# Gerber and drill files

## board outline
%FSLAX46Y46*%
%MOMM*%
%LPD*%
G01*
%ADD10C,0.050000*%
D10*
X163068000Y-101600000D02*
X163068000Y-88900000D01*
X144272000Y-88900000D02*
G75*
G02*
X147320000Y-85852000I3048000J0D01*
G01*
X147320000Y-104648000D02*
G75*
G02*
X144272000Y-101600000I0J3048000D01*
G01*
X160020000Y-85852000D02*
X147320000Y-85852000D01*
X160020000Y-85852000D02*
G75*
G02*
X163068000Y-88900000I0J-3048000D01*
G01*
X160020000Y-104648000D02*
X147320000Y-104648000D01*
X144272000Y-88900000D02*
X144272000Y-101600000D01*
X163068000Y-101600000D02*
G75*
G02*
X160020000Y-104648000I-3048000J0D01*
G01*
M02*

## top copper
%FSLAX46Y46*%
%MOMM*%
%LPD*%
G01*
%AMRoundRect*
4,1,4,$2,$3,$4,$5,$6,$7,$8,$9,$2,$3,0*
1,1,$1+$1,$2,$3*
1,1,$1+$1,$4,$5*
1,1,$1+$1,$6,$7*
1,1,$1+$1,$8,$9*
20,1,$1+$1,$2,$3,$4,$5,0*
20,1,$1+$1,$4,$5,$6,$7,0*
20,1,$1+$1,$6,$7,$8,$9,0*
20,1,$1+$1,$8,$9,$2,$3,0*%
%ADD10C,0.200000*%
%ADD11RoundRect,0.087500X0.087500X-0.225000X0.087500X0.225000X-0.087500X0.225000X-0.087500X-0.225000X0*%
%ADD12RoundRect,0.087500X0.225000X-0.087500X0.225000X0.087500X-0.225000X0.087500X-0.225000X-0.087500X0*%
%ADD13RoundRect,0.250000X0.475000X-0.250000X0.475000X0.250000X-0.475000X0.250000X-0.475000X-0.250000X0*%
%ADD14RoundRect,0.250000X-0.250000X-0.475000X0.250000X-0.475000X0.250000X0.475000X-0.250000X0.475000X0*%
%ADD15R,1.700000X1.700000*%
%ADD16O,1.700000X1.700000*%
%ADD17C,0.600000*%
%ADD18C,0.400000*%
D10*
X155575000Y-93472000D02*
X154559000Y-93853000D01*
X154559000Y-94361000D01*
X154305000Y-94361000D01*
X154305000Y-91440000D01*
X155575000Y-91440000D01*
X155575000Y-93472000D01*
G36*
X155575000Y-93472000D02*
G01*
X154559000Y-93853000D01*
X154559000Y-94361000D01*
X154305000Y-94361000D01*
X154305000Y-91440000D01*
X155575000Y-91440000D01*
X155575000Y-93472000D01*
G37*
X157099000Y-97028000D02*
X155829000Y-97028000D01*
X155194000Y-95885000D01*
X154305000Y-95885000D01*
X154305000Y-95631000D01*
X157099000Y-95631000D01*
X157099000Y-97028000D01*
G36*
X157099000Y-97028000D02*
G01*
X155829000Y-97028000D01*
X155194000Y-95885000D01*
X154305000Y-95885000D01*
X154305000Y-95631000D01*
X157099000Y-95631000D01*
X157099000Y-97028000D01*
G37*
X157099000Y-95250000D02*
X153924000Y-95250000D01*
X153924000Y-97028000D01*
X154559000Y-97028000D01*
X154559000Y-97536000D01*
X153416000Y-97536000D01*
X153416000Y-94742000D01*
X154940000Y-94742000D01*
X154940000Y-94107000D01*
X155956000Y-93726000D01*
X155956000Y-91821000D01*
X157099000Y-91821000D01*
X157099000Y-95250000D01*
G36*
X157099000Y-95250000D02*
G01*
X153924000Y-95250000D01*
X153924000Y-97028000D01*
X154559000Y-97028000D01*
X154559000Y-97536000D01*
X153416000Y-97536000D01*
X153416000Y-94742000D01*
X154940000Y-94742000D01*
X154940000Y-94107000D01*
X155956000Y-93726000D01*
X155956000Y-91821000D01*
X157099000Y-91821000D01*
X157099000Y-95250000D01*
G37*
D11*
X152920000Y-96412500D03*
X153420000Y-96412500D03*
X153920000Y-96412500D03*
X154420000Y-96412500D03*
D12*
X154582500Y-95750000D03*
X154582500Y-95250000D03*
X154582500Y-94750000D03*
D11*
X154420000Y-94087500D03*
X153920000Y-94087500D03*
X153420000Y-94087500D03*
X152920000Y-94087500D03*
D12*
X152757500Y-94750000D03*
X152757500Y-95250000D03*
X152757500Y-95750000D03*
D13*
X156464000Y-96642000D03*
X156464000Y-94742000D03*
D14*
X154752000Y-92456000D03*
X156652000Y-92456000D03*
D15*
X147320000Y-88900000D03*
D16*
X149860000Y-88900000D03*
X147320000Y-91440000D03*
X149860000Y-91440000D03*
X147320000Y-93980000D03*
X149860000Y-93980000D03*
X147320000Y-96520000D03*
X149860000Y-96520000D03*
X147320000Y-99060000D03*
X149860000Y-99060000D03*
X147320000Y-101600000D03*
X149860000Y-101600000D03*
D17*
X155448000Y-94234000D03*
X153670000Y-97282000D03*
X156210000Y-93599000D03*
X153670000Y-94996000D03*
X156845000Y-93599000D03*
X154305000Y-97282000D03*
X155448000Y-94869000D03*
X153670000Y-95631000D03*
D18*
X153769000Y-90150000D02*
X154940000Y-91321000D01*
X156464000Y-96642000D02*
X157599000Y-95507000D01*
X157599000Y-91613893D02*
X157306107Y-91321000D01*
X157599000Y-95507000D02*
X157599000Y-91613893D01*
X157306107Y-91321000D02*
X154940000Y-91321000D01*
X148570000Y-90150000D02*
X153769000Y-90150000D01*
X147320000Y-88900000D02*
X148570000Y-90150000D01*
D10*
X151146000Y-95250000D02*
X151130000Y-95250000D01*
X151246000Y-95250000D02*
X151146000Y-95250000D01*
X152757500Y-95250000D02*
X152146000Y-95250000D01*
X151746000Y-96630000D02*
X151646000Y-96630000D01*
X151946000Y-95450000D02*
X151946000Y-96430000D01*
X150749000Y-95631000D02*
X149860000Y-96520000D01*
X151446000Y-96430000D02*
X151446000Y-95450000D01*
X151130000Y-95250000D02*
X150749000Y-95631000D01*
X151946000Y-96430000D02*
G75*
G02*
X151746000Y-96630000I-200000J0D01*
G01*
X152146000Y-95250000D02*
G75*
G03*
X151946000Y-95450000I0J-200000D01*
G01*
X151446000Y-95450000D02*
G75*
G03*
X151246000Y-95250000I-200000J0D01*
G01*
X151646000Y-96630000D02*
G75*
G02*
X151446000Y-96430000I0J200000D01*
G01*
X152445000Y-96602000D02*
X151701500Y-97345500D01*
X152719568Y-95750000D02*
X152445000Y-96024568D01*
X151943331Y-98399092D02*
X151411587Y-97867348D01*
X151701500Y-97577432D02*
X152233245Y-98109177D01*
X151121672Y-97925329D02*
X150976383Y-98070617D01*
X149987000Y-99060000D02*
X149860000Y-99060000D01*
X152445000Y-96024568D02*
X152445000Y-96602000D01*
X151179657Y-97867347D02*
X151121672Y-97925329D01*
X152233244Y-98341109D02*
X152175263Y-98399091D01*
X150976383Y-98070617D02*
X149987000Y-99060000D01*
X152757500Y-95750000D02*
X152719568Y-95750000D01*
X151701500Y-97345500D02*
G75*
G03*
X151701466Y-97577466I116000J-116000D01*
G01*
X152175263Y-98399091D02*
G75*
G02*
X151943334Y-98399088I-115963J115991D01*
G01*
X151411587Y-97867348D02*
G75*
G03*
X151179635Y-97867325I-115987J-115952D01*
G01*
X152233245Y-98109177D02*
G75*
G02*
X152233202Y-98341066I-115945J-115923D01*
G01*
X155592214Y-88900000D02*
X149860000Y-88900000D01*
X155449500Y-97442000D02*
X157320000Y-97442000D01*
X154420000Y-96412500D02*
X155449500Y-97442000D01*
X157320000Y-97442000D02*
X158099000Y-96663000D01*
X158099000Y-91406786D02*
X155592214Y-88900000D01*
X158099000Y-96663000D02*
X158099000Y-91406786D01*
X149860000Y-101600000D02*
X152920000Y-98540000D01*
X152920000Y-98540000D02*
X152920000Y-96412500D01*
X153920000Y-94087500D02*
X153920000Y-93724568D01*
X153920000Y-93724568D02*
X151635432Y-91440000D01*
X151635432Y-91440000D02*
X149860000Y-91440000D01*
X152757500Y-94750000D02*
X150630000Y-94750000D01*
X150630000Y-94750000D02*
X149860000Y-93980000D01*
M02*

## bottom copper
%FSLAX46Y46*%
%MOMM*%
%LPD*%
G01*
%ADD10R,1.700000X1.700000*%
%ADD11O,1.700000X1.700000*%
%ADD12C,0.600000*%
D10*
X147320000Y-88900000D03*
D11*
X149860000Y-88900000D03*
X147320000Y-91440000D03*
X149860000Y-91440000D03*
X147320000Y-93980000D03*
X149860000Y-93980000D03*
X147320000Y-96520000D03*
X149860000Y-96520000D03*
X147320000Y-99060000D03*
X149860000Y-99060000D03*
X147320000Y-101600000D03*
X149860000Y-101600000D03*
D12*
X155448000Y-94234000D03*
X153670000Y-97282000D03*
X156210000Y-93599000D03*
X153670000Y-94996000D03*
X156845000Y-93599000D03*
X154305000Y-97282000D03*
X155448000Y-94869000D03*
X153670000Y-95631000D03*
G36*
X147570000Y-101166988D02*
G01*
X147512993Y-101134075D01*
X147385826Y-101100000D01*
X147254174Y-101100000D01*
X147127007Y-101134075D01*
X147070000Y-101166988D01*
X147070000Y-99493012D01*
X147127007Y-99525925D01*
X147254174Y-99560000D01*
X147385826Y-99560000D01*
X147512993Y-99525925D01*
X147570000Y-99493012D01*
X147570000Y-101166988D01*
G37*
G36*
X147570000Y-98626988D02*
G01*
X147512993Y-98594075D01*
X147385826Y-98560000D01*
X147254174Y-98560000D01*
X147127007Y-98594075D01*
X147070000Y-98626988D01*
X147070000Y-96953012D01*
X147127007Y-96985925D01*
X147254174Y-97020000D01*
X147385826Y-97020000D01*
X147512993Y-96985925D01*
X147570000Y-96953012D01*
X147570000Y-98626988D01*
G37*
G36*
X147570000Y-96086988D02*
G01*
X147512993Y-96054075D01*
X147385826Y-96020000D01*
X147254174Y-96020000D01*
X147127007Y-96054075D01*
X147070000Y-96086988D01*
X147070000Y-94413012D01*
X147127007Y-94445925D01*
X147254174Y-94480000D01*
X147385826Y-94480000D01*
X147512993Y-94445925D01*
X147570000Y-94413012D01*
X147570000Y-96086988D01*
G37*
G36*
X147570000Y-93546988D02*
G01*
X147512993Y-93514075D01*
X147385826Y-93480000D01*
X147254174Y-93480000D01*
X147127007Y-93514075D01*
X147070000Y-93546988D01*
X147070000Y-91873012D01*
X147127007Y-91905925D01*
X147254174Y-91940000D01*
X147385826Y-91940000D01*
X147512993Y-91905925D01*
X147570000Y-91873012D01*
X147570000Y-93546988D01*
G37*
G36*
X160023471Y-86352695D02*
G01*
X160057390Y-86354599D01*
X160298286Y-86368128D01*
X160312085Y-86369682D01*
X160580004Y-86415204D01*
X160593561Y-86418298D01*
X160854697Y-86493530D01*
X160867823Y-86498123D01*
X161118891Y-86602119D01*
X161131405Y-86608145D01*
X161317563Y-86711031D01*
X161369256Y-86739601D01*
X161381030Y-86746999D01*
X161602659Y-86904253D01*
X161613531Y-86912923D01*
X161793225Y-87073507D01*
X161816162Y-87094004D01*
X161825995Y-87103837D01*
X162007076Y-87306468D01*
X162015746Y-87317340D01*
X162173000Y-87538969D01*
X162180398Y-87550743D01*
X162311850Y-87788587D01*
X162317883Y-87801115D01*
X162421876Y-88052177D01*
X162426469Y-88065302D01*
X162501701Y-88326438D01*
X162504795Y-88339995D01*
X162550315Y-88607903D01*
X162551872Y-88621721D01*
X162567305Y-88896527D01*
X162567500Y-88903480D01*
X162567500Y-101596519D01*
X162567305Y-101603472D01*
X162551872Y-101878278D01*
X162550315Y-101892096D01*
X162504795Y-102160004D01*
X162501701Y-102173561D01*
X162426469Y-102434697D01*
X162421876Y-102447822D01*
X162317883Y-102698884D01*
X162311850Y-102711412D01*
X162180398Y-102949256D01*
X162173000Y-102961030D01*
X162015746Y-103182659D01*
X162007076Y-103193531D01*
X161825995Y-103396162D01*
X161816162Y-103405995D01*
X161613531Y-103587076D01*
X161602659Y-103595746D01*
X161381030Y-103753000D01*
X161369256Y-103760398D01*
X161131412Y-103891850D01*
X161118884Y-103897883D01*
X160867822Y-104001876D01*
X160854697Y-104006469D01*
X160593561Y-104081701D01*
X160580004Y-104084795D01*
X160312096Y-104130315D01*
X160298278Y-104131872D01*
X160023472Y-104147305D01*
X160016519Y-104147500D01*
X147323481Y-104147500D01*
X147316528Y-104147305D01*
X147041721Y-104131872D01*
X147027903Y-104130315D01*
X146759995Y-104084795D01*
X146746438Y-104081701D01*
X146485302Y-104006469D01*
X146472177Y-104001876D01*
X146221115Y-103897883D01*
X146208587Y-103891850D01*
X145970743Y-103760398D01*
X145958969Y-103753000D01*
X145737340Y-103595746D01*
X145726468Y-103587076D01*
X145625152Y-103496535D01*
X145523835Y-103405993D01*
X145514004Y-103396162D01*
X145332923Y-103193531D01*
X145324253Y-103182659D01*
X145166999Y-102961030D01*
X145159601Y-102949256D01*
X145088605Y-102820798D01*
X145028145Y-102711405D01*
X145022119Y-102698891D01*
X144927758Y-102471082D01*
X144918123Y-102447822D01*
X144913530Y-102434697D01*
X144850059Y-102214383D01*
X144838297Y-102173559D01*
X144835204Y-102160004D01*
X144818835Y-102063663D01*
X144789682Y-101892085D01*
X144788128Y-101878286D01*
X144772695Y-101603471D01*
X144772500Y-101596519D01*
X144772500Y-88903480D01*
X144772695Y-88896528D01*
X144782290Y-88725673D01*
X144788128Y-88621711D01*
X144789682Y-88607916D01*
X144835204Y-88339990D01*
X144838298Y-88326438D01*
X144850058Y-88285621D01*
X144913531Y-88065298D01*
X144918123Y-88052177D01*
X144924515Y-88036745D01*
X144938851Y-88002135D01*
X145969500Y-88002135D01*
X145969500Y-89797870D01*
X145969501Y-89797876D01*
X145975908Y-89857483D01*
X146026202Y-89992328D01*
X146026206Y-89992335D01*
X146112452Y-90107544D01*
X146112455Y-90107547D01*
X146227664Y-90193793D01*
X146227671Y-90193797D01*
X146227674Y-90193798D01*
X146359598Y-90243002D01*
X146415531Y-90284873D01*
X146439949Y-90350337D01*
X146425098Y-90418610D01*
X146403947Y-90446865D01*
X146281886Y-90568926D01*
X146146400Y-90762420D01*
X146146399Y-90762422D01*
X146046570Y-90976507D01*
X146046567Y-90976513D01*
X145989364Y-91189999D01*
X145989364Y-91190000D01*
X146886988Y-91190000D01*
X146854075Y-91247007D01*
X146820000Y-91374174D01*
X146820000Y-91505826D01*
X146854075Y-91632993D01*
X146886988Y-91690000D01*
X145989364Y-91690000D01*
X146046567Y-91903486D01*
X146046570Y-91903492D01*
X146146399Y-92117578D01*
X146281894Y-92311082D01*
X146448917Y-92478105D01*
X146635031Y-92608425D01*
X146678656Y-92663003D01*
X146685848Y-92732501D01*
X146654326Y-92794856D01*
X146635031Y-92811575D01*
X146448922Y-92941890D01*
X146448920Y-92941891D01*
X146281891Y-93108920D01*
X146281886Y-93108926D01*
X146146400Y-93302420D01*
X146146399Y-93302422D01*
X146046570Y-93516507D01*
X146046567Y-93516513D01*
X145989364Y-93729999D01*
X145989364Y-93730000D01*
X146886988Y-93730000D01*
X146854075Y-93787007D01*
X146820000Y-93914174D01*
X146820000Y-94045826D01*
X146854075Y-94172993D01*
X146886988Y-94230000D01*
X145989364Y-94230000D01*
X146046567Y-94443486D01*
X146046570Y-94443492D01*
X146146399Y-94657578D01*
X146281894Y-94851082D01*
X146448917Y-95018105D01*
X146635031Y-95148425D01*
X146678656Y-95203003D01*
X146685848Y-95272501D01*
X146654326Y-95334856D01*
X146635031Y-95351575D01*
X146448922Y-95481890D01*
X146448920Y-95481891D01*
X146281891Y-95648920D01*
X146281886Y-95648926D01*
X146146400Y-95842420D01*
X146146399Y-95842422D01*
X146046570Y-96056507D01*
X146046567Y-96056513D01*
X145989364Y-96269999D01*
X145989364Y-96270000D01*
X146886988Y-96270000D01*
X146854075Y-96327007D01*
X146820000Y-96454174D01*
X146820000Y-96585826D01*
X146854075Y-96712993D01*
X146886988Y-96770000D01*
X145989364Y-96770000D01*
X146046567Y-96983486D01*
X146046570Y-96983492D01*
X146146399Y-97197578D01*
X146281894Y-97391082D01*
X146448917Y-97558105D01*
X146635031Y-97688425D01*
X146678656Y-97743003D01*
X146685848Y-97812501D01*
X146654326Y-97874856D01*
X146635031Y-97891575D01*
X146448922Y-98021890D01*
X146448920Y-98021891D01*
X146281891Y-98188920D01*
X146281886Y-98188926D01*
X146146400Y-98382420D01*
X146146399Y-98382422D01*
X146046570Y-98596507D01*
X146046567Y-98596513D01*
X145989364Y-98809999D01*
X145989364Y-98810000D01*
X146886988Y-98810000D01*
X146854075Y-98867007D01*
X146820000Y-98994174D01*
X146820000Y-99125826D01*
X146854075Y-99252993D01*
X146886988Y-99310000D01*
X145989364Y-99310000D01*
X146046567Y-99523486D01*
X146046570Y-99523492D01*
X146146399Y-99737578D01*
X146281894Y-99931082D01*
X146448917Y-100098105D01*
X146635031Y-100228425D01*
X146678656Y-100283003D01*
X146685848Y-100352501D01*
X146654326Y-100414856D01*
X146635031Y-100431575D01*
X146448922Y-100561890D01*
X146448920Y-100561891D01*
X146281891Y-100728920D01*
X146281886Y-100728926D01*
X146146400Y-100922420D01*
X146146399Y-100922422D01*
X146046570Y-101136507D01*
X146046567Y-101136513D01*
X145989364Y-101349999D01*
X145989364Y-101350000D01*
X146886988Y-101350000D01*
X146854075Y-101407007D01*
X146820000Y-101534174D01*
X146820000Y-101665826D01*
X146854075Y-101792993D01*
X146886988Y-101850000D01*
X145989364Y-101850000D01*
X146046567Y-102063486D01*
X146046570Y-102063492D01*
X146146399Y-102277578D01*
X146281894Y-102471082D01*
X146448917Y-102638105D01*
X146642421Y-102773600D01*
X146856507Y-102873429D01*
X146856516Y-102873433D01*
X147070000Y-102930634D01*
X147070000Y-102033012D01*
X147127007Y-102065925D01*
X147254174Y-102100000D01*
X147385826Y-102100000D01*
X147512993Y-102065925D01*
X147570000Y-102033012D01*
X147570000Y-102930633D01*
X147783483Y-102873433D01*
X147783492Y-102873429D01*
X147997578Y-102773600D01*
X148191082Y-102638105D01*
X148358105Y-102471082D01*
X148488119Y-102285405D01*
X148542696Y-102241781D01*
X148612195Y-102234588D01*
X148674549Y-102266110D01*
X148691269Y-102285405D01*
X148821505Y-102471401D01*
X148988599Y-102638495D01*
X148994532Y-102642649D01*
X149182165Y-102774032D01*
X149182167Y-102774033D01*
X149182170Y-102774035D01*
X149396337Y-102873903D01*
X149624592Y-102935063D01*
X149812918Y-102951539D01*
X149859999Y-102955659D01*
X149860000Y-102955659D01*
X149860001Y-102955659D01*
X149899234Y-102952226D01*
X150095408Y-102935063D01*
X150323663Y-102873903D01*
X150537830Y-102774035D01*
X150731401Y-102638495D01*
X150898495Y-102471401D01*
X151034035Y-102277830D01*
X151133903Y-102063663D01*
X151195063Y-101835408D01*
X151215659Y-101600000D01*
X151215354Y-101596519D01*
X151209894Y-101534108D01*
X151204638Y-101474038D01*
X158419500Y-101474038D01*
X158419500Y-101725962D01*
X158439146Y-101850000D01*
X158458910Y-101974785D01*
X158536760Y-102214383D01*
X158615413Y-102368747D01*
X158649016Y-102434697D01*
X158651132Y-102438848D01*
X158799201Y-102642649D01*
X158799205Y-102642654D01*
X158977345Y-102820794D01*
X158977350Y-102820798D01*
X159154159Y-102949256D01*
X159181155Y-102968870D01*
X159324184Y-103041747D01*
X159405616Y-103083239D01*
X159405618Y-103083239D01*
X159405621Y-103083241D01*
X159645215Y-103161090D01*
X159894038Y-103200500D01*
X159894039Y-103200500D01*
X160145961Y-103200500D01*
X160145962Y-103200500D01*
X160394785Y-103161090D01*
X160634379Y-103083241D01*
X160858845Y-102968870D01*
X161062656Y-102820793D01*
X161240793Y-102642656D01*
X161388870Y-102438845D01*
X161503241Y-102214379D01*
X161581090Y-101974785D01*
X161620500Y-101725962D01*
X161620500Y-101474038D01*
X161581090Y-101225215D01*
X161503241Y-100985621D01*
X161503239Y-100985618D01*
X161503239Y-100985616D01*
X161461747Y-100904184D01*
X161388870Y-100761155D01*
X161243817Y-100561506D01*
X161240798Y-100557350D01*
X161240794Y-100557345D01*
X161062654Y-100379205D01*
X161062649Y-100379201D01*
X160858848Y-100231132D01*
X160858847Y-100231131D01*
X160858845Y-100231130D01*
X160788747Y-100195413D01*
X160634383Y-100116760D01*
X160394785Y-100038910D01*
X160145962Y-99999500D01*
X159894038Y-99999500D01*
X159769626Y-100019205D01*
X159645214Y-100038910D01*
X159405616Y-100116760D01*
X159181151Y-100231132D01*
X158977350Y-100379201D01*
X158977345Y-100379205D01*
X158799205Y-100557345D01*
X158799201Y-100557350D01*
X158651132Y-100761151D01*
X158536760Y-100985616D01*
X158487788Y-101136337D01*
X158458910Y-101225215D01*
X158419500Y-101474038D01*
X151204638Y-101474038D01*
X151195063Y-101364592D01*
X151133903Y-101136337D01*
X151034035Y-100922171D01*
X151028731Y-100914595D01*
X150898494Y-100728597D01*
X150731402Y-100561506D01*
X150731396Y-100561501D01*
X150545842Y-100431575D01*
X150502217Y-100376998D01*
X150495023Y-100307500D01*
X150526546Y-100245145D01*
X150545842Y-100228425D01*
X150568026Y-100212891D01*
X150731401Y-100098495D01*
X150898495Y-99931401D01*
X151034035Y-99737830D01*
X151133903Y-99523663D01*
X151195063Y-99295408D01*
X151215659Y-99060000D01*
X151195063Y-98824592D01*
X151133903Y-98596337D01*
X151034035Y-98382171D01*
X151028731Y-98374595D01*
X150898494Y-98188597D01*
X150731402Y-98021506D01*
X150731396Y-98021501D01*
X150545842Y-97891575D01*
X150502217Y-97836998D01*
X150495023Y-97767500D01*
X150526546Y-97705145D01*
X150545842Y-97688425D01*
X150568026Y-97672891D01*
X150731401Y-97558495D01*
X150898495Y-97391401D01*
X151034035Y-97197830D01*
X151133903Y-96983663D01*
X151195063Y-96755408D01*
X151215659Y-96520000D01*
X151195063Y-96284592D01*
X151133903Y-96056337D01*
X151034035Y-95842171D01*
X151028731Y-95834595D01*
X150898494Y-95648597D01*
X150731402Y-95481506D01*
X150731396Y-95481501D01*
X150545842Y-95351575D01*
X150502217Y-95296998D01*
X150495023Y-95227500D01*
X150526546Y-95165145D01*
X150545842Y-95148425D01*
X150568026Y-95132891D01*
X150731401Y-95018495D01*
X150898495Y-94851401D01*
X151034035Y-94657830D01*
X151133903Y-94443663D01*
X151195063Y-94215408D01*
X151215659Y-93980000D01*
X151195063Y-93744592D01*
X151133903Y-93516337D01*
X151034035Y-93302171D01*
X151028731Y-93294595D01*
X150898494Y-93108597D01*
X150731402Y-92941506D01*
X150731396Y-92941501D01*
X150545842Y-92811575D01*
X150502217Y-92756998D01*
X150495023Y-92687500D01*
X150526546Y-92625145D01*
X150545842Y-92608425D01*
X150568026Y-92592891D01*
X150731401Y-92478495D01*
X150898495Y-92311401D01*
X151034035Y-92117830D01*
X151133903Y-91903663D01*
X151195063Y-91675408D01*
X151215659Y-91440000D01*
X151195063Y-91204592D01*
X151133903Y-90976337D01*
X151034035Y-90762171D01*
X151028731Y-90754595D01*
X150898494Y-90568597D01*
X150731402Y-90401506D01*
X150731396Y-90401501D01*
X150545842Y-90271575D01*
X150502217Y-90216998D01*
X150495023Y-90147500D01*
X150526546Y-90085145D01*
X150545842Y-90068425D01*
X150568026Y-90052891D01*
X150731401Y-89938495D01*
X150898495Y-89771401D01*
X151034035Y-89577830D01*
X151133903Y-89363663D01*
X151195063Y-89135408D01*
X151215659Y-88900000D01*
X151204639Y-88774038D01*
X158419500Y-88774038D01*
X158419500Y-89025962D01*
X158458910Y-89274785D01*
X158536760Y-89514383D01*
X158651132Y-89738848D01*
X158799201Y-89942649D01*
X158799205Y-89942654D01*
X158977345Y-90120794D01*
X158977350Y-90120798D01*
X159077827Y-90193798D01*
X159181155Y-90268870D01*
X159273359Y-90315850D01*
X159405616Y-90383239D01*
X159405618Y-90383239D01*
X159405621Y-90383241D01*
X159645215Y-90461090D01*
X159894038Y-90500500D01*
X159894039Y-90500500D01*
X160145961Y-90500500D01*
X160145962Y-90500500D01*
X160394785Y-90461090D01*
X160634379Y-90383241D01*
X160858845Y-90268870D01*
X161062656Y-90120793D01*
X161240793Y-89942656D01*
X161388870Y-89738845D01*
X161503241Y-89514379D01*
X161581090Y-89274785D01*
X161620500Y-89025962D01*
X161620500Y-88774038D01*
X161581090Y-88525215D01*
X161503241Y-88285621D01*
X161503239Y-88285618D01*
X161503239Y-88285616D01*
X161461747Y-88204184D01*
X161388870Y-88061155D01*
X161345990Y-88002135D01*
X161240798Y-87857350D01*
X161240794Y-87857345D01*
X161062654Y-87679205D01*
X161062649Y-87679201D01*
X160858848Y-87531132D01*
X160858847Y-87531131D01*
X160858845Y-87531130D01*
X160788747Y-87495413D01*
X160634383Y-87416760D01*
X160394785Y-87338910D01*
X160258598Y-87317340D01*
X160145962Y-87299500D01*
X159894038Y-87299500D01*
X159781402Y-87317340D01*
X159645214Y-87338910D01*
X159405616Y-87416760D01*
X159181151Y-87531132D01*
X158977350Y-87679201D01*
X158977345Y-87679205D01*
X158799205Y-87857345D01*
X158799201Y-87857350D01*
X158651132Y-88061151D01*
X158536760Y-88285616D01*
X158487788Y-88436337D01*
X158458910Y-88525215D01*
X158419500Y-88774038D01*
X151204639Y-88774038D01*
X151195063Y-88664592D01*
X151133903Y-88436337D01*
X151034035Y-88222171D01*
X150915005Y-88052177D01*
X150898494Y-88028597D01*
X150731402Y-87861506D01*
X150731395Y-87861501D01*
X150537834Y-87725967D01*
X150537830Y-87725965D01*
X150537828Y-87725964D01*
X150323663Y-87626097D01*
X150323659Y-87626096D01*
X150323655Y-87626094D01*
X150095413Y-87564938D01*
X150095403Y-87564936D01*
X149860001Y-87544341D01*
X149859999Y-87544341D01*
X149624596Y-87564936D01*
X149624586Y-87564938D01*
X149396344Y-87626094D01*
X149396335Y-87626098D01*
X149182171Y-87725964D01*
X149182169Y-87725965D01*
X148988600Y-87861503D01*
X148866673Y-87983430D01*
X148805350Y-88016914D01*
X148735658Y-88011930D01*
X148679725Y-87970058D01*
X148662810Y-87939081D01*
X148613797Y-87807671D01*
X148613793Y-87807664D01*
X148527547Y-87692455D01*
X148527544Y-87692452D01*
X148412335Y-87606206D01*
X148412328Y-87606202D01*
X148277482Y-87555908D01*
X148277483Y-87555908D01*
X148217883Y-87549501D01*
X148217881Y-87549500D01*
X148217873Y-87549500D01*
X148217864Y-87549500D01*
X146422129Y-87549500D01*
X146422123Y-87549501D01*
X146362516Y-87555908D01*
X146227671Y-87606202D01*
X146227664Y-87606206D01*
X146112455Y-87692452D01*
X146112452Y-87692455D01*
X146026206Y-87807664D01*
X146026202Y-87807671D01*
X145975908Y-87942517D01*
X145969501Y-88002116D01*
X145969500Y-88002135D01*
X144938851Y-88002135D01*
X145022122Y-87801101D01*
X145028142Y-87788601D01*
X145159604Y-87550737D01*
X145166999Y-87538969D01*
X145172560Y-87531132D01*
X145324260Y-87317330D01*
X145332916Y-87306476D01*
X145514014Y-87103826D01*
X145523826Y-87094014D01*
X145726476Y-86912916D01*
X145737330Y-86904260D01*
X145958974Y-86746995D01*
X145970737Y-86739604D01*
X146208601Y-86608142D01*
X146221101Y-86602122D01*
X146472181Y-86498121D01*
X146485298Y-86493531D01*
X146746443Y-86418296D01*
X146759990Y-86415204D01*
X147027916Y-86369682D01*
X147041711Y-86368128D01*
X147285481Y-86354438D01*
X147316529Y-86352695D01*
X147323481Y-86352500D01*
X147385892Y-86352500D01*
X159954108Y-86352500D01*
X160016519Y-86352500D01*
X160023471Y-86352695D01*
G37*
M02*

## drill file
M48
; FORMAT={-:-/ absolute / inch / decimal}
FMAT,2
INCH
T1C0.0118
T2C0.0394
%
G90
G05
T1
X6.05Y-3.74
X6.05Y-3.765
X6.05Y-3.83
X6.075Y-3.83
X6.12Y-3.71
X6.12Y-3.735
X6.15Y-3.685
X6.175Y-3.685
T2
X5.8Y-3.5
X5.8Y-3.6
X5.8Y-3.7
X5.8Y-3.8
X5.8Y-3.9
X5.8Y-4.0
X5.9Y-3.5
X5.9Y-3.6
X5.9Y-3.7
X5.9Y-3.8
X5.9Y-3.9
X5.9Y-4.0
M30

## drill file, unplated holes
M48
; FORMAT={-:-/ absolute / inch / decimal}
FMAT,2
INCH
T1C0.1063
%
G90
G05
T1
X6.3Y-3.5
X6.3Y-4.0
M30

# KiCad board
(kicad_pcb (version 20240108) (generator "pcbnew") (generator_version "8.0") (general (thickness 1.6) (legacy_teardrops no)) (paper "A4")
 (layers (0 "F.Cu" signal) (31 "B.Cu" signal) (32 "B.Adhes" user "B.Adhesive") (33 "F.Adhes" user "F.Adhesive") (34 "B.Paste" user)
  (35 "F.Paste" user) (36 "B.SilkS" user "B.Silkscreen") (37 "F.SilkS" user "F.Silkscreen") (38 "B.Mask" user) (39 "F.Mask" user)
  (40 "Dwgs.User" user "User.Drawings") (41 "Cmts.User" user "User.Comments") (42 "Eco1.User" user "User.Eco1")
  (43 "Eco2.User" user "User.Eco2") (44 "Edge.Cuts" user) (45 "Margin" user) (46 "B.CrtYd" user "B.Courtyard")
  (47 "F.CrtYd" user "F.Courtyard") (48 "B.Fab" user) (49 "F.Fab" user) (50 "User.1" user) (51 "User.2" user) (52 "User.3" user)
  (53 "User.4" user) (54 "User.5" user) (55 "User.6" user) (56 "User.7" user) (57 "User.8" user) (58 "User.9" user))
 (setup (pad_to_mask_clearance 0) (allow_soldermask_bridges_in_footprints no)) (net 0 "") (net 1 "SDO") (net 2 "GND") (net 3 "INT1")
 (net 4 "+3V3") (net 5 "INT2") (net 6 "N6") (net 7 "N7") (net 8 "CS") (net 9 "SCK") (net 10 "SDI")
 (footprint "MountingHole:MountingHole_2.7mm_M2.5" (layer "F.Cu") (at 160.02 101.6)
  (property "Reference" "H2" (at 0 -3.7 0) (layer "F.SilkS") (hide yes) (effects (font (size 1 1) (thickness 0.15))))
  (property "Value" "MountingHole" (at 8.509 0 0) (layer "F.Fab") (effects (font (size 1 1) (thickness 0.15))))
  (pad "" np_thru_hole circle (at 0 0) (size 2.7 2.7) (drill 2.7) (layers "*.Cu" "*.Mask")))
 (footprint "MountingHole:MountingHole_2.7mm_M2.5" (layer "F.Cu") (at 160.02 88.9)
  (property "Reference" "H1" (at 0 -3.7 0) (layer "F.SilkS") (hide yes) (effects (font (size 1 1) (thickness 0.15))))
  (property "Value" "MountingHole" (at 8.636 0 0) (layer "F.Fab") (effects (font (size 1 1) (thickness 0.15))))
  (pad "" np_thru_hole circle (at 0 0) (size 2.7 2.7) (drill 2.7) (layers "*.Cu" "*.Mask")))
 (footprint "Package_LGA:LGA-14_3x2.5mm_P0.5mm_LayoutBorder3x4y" (layer "F.Cu") (at 153.67 95.25 90)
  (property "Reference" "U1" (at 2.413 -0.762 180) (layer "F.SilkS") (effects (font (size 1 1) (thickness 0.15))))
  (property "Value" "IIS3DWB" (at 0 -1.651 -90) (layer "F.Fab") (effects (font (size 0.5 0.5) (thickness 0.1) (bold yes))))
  (pad "1" smd roundrect (at -1.1625 -0.75 90) (size 0.625 0.35) (layers "F.Cu" "F.Paste" "F.Mask") (roundrect_rratio 0.25) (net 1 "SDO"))
  (pad "2" smd roundrect (at -1.1625 -0.25 90) (size 0.625 0.35) (layers "F.Cu" "F.Paste" "F.Mask") (roundrect_rratio 0.25) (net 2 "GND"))
  (pad "3" smd roundrect (at -1.1625 0.25 90) (size 0.625 0.35) (layers "F.Cu" "F.Paste" "F.Mask") (roundrect_rratio 0.25) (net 2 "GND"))
  (pad "4" smd roundrect (at -1.1625 0.75 90) (size 0.625 0.35) (layers "F.Cu" "F.Paste" "F.Mask") (roundrect_rratio 0.25) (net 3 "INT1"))
  (pad "5" smd roundrect (at -0.5 0.9125 90) (size 0.35 0.625) (layers "F.Cu" "F.Paste" "F.Mask") (roundrect_rratio 0.25) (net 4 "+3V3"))
  (pad "6" smd roundrect (at 0 0.9125 90) (size 0.35 0.625) (layers "F.Cu" "F.Paste" "F.Mask") (roundrect_rratio 0.25) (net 2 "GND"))
  (pad "7" smd roundrect (at 0.5 0.9125 90) (size 0.35 0.625) (layers "F.Cu" "F.Paste" "F.Mask") (roundrect_rratio 0.25) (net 2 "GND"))
  (pad "8" smd roundrect (at 1.1625 0.75 90) (size 0.625 0.35) (layers "F.Cu" "F.Paste" "F.Mask") (roundrect_rratio 0.25) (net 4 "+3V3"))
  (pad "9" smd roundrect (at 1.1625 0.25 90) (size 0.625 0.35) (layers "F.Cu" "F.Paste" "F.Mask") (roundrect_rratio 0.25) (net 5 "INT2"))
  (pad "10" smd roundrect (at 1.1625 -0.25 90) (size 0.625 0.35) (layers "F.Cu" "F.Paste" "F.Mask") (roundrect_rratio 0.25) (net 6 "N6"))
  (pad "11" smd roundrect (at 1.1625 -0.75 90) (size 0.625 0.35) (layers "F.Cu" "F.Paste" "F.Mask") (roundrect_rratio 0.25) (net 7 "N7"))
  (pad "12" smd roundrect (at 0.5 -0.9125 90) (size 0.35 0.625) (layers "F.Cu" "F.Paste" "F.Mask") (roundrect_rratio 0.25) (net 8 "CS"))
  (pad "13" smd roundrect (at 0 -0.9125 90) (size 0.35 0.625) (layers "F.Cu" "F.Paste" "F.Mask") (roundrect_rratio 0.25) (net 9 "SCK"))
  (pad "14" smd roundrect (at -0.5 -0.9125 90) (size 0.35 0.625) (layers "F.Cu" "F.Paste" "F.Mask") (roundrect_rratio 0.25) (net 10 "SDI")))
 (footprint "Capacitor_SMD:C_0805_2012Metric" (layer "F.Cu") (at 156.464 95.692 90)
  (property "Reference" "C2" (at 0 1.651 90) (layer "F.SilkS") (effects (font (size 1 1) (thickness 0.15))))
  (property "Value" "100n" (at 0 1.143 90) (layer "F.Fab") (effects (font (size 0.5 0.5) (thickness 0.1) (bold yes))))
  (pad "1" smd roundrect (at -0.95 0 90) (size 1 1.45) (layers "F.Cu" "F.Paste" "F.Mask") (roundrect_rratio 0.25) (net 4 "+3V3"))
  (pad "2" smd roundrect (at 0.95 0 90) (size 1 1.45) (layers "F.Cu" "F.Paste" "F.Mask") (roundrect_rratio 0.25) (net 2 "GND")))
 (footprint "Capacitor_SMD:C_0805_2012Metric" (layer "F.Cu") (at 155.702 92.456)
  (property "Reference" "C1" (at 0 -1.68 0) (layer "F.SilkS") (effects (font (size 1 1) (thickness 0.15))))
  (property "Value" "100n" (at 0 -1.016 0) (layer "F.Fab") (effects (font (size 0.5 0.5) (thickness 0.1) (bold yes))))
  (pad "1" smd roundrect (at -0.95 0) (size 1 1.45) (layers "F.Cu" "F.Paste" "F.Mask") (roundrect_rratio 0.25) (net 4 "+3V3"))
  (pad "2" smd roundrect (at 0.95 0) (size 1 1.45) (layers "F.Cu" "F.Paste" "F.Mask") (roundrect_rratio 0.25) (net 2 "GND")))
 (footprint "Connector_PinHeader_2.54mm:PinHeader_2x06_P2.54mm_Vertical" (layer "F.Cu") (at 147.32 88.9)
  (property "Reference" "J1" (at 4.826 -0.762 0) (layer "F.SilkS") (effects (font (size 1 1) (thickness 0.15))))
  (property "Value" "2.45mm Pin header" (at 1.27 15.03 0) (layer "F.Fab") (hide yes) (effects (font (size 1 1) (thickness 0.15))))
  (pad "1" thru_hole rect (at 0 0) (size 1.7 1.7) (drill 1) (layers "*.Cu" "*.Mask") (remove_unused_layers no) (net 4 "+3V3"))
  (pad "2" thru_hole oval (at 2.54 0) (size 1.7 1.7) (drill 1) (layers "*.Cu" "*.Mask") (remove_unused_layers no) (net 3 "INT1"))
  (pad "3" thru_hole oval (at 0 2.54) (size 1.7 1.7) (drill 1) (layers "*.Cu" "*.Mask") (remove_unused_layers no) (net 2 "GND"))
  (pad "4" thru_hole oval (at 2.54 2.54) (size 1.7 1.7) (drill 1) (layers "*.Cu" "*.Mask") (remove_unused_layers no) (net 5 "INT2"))
  (pad "5" thru_hole oval (at 0 5.08) (size 1.7 1.7) (drill 1) (layers "*.Cu" "*.Mask") (remove_unused_layers no) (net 2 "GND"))
  (pad "6" thru_hole oval (at 2.54 5.08) (size 1.7 1.7) (drill 1) (layers "*.Cu" "*.Mask") (remove_unused_layers no) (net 8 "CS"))
  (pad "7" thru_hole oval (at 0 7.62) (size 1.7 1.7) (drill 1) (layers "*.Cu" "*.Mask") (remove_unused_layers no) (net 2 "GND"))
  (pad "8" thru_hole oval (at 2.54 7.62) (size 1.7 1.7) (drill 1) (layers "*.Cu" "*.Mask") (remove_unused_layers no) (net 9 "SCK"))
  (pad "9" thru_hole oval (at 0 10.16) (size 1.7 1.7) (drill 1) (layers "*.Cu" "*.Mask") (remove_unused_layers no) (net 2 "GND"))
  (pad "10" thru_hole oval (at 2.54 10.16) (size 1.7 1.7) (drill 1) (layers "*.Cu" "*.Mask") (remove_unused_layers no) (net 10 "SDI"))
  (pad "11" thru_hole oval (at 0 12.7) (size 1.7 1.7) (drill 1) (layers "*.Cu" "*.Mask") (remove_unused_layers no) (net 2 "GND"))
  (pad "12" thru_hole oval (at 2.54 12.7) (size 1.7 1.7) (drill 1) (layers "*.Cu" "*.Mask") (remove_unused_layers no) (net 1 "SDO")))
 (gr_poly
  (pts (xy 154.305 94.361) (xy 154.305 91.44) (xy 155.575 91.44) (xy 155.575 93.472) (xy 154.559 93.853) (xy 154.559 94.361))
  (stroke (width 0.2) (type solid)) (fill solid) (layer "F.Cu") (net 4))
 (gr_poly
  (pts (xy 154.305 95.631) (xy 157.099 95.631) (xy 157.099 97.028) (xy 155.829 97.028) (xy 155.194 95.885) (xy 154.305 95.885))
  (stroke (width 0.2) (type solid)) (fill solid) (layer "F.Cu") (net 4))
 (gr_poly
  (pts (xy 153.416 94.742) (xy 153.416 97.536) (xy 154.559 97.536) (xy 154.559 97.028) (xy 153.924 97.028) (xy 153.924 95.25)
   (xy 157.099 95.25) (xy 157.099 91.821) (xy 155.956 91.821) (xy 155.956 93.726) (xy 154.94 94.107) (xy 154.94 94.742))
  (stroke (width 0.2) (type solid)) (fill solid) (layer "F.Cu") (net 2))
 (gr_line (start 163.068 101.6) (end 163.068 88.9) (stroke (width 0.05) (type default)) (layer "Edge.Cuts"))
 (gr_arc (start 144.272 88.9) (mid 145.164739 86.744739) (end 147.32 85.852) (stroke (width 0.05) (type default)) (layer "Edge.Cuts"))
 (gr_arc (start 147.32 104.648) (mid 145.164739 103.755261) (end 144.272 101.6) (stroke (width 0.05) (type default)) (layer "Edge.Cuts"))
 (gr_line (start 160.02 85.852) (end 147.32 85.852) (stroke (width 0.05) (type default)) (layer "Edge.Cuts"))
 (gr_arc (start 160.02 85.852) (mid 162.175261 86.744739) (end 163.068 88.9) (stroke (width 0.05) (type default)) (layer "Edge.Cuts"))
 (gr_line (start 160.02 104.648) (end 147.32 104.648) (stroke (width 0.05) (type default)) (layer "Edge.Cuts"))
 (gr_line (start 144.272 88.9) (end 144.272 101.6) (stroke (width 0.05) (type default)) (layer "Edge.Cuts"))
 (gr_arc (start 163.068 101.6) (mid 162.175261 103.755261) (end 160.02 104.648) (stroke (width 0.05) (type default)) (layer "Edge.Cuts"))
 (via (at 155.448 94.234) (size 0.6) (drill 0.3) (layers "F.Cu" "B.Cu") (free yes) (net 2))
 (via (at 153.67 97.282) (size 0.6) (drill 0.3) (layers "F.Cu" "B.Cu") (free yes) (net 2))
 (via (at 156.21 93.599) (size 0.6) (drill 0.3) (layers "F.Cu" "B.Cu") (free yes) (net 2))
 (via (at 153.67 94.996) (size 0.6) (drill 0.3) (layers "F.Cu" "B.Cu") (free yes) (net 2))
 (via (at 156.845 93.599) (size 0.6) (drill 0.3) (layers "F.Cu" "B.Cu") (free yes) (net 2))
 (via (at 154.305 97.282) (size 0.6) (drill 0.3) (layers "F.Cu" "B.Cu") (free yes) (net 2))
 (via (at 155.448 94.869) (size 0.6) (drill 0.3) (layers "F.Cu" "B.Cu") (free yes) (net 2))
 (via (at 153.67 95.631) (size 0.6) (drill 0.3) (layers "F.Cu" "B.Cu") (free yes) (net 2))
 (segment (start 147.32 88.9) (end 148.59 90.17) (width 0.4) (layer "F.Cu") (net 4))
 (segment (start 157.306107 91.321) (end 157.599 91.613893) (width 0.4) (layer "F.Cu") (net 4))
 (segment (start 148.59 90.17) (end 153.035 90.17) (width 0.4) (layer "F.Cu") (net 4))
 (segment (start 157.599 95.507) (end 156.464 96.642) (width 0.4) (layer "F.Cu") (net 4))
 (segment (start 157.599 91.613893) (end 157.599 95.507) (width 0.4) (layer "F.Cu") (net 4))
 (segment (start 153.035 90.17) (end 154.186 91.321) (width 0.4) (layer "F.Cu") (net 4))
 (segment (start 154.186 91.321) (end 157.306107 91.321) (width 0.4) (layer "F.Cu") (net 4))
 (segment (start 151.146 95.25) (end 151.13 95.25) (width 0.2) (layer "F.Cu") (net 9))
 (segment (start 151.246 95.25) (end 151.146 95.25) (width 0.2) (layer "F.Cu") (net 9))
 (segment (start 152.7575 95.25) (end 152.146 95.25) (width 0.2) (layer "F.Cu") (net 9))
 (segment (start 151.746 96.63) (end 151.646 96.63) (width 0.2) (layer "F.Cu") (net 9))
 (segment (start 151.946 95.45) (end 151.946 96.43) (width 0.2) (layer "F.Cu") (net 9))
 (segment (start 150.749 95.631) (end 149.86 96.52) (width 0.2) (layer "F.Cu") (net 9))
 (segment (start 151.446 96.43) (end 151.446 95.45) (width 0.2) (layer "F.Cu") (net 9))
 (segment (start 151.13 95.25) (end 150.749 95.631) (width 0.2) (layer "F.Cu") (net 9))
 (arc (start 151.946 96.43) (mid 151.887421 96.571421) (end 151.746 96.63) (width 0.2) (layer "F.Cu") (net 9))
 (arc (start 152.146 95.25) (mid 152.004579 95.308579) (end 151.946 95.45) (width 0.2) (layer "F.Cu") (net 9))
 (arc (start 151.446 95.45) (mid 151.387421 95.308579) (end 151.246 95.25) (width 0.2) (layer "F.Cu") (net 9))
 (arc (start 151.646 96.63) (mid 151.504579 96.571421) (end 151.446 96.43) (width 0.2) (layer "F.Cu") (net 9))
 (segment (start 152.445 96.602) (end 151.7015 97.3455) (width 0.2) (layer "F.Cu") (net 10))
 (segment (start 152.719568 95.75) (end 152.445 96.024568) (width 0.2) (layer "F.Cu") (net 10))
 (segment (start 151.943331 98.399092) (end 151.411587 97.867348) (width 0.2) (layer "F.Cu") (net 10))
 (segment (start 151.7015 97.577432) (end 152.233245 98.109177) (width 0.2) (layer "F.Cu") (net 10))
 (segment (start 151.121672 97.925329) (end 150.976383 98.070617) (width 0.2) (layer "F.Cu") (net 10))
 (segment (start 149.987 99.06) (end 149.86 99.06) (width 0.2) (layer "F.Cu") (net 10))
 (segment (start 152.445 96.024568) (end 152.445 96.602) (width 0.2) (layer "F.Cu") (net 10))
 (segment (start 151.179657 97.867347) (end 151.121672 97.925329) (width 0.2) (layer "F.Cu") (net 10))
 (segment (start 152.233244 98.341109) (end 152.175263 98.399091) (width 0.2) (layer "F.Cu") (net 10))
 (segment (start 150.976383 98.070617) (end 149.987 99.06) (width 0.2) (layer "F.Cu") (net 10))
 (segment (start 152.7575 95.75) (end 152.719568 95.75) (width 0.2) (layer "F.Cu") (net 10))
 (arc (start 151.7015 97.3455) (mid 151.653464 97.461467) (end 151.7015 97.577432) (width 0.2) (layer "F.Cu") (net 10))
 (arc (start 152.175263 98.399091) (mid 152.059297 98.447126) (end 151.943331 98.399092) (width 0.2) (layer "F.Cu") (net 10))
 (arc (start 151.411587 97.867348) (mid 151.295621 97.819314) (end 151.179657 97.867347) (width 0.2) (layer "F.Cu") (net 10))
 (arc (start 152.233245 98.109177) (mid 152.28128 98.225142) (end 152.233244 98.341109) (width 0.2) (layer "F.Cu") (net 10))
 (segment (start 155.592214 88.9) (end 149.86 88.9) (width 0.2) (layer "F.Cu") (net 3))
 (segment (start 155.4495 97.442) (end 157.32 97.442) (width 0.2) (layer "F.Cu") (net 3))
 (segment (start 154.42 96.4125) (end 155.4495 97.442) (width 0.2) (layer "F.Cu") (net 3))
 (segment (start 157.32 97.442) (end 158.099 96.663) (width 0.2) (layer "F.Cu") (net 3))
 (segment (start 158.099 91.406786) (end 155.592214 88.9) (width 0.2) (layer "F.Cu") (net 3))
 (segment (start 158.099 96.663) (end 158.099 91.406786) (width 0.2) (layer "F.Cu") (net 3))
 (segment (start 149.86 101.6) (end 152.92 98.54) (width 0.2) (layer "F.Cu") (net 1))
 (segment (start 152.92 98.54) (end 152.92 96.4125) (width 0.2) (layer "F.Cu") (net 1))
 (segment (start 153.92 94.0875) (end 153.92 93.724568) (width 0.2) (layer "F.Cu") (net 5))
 (segment (start 153.92 93.724568) (end 151.635432 91.44) (width 0.2) (layer "F.Cu") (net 5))
 (segment (start 151.635432 91.44) (end 149.86 91.44) (width 0.2) (layer "F.Cu") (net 5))
 (segment (start 152.7575 94.75) (end 150.63 94.75) (width 0.2) (layer "F.Cu") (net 8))
 (segment (start 150.63 94.75) (end 149.86 93.98) (width 0.2) (layer "F.Cu") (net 8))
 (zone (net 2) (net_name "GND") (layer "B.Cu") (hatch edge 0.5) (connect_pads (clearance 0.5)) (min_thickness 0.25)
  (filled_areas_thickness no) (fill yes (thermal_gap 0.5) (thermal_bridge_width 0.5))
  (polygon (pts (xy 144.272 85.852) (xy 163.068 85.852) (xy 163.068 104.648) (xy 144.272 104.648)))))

